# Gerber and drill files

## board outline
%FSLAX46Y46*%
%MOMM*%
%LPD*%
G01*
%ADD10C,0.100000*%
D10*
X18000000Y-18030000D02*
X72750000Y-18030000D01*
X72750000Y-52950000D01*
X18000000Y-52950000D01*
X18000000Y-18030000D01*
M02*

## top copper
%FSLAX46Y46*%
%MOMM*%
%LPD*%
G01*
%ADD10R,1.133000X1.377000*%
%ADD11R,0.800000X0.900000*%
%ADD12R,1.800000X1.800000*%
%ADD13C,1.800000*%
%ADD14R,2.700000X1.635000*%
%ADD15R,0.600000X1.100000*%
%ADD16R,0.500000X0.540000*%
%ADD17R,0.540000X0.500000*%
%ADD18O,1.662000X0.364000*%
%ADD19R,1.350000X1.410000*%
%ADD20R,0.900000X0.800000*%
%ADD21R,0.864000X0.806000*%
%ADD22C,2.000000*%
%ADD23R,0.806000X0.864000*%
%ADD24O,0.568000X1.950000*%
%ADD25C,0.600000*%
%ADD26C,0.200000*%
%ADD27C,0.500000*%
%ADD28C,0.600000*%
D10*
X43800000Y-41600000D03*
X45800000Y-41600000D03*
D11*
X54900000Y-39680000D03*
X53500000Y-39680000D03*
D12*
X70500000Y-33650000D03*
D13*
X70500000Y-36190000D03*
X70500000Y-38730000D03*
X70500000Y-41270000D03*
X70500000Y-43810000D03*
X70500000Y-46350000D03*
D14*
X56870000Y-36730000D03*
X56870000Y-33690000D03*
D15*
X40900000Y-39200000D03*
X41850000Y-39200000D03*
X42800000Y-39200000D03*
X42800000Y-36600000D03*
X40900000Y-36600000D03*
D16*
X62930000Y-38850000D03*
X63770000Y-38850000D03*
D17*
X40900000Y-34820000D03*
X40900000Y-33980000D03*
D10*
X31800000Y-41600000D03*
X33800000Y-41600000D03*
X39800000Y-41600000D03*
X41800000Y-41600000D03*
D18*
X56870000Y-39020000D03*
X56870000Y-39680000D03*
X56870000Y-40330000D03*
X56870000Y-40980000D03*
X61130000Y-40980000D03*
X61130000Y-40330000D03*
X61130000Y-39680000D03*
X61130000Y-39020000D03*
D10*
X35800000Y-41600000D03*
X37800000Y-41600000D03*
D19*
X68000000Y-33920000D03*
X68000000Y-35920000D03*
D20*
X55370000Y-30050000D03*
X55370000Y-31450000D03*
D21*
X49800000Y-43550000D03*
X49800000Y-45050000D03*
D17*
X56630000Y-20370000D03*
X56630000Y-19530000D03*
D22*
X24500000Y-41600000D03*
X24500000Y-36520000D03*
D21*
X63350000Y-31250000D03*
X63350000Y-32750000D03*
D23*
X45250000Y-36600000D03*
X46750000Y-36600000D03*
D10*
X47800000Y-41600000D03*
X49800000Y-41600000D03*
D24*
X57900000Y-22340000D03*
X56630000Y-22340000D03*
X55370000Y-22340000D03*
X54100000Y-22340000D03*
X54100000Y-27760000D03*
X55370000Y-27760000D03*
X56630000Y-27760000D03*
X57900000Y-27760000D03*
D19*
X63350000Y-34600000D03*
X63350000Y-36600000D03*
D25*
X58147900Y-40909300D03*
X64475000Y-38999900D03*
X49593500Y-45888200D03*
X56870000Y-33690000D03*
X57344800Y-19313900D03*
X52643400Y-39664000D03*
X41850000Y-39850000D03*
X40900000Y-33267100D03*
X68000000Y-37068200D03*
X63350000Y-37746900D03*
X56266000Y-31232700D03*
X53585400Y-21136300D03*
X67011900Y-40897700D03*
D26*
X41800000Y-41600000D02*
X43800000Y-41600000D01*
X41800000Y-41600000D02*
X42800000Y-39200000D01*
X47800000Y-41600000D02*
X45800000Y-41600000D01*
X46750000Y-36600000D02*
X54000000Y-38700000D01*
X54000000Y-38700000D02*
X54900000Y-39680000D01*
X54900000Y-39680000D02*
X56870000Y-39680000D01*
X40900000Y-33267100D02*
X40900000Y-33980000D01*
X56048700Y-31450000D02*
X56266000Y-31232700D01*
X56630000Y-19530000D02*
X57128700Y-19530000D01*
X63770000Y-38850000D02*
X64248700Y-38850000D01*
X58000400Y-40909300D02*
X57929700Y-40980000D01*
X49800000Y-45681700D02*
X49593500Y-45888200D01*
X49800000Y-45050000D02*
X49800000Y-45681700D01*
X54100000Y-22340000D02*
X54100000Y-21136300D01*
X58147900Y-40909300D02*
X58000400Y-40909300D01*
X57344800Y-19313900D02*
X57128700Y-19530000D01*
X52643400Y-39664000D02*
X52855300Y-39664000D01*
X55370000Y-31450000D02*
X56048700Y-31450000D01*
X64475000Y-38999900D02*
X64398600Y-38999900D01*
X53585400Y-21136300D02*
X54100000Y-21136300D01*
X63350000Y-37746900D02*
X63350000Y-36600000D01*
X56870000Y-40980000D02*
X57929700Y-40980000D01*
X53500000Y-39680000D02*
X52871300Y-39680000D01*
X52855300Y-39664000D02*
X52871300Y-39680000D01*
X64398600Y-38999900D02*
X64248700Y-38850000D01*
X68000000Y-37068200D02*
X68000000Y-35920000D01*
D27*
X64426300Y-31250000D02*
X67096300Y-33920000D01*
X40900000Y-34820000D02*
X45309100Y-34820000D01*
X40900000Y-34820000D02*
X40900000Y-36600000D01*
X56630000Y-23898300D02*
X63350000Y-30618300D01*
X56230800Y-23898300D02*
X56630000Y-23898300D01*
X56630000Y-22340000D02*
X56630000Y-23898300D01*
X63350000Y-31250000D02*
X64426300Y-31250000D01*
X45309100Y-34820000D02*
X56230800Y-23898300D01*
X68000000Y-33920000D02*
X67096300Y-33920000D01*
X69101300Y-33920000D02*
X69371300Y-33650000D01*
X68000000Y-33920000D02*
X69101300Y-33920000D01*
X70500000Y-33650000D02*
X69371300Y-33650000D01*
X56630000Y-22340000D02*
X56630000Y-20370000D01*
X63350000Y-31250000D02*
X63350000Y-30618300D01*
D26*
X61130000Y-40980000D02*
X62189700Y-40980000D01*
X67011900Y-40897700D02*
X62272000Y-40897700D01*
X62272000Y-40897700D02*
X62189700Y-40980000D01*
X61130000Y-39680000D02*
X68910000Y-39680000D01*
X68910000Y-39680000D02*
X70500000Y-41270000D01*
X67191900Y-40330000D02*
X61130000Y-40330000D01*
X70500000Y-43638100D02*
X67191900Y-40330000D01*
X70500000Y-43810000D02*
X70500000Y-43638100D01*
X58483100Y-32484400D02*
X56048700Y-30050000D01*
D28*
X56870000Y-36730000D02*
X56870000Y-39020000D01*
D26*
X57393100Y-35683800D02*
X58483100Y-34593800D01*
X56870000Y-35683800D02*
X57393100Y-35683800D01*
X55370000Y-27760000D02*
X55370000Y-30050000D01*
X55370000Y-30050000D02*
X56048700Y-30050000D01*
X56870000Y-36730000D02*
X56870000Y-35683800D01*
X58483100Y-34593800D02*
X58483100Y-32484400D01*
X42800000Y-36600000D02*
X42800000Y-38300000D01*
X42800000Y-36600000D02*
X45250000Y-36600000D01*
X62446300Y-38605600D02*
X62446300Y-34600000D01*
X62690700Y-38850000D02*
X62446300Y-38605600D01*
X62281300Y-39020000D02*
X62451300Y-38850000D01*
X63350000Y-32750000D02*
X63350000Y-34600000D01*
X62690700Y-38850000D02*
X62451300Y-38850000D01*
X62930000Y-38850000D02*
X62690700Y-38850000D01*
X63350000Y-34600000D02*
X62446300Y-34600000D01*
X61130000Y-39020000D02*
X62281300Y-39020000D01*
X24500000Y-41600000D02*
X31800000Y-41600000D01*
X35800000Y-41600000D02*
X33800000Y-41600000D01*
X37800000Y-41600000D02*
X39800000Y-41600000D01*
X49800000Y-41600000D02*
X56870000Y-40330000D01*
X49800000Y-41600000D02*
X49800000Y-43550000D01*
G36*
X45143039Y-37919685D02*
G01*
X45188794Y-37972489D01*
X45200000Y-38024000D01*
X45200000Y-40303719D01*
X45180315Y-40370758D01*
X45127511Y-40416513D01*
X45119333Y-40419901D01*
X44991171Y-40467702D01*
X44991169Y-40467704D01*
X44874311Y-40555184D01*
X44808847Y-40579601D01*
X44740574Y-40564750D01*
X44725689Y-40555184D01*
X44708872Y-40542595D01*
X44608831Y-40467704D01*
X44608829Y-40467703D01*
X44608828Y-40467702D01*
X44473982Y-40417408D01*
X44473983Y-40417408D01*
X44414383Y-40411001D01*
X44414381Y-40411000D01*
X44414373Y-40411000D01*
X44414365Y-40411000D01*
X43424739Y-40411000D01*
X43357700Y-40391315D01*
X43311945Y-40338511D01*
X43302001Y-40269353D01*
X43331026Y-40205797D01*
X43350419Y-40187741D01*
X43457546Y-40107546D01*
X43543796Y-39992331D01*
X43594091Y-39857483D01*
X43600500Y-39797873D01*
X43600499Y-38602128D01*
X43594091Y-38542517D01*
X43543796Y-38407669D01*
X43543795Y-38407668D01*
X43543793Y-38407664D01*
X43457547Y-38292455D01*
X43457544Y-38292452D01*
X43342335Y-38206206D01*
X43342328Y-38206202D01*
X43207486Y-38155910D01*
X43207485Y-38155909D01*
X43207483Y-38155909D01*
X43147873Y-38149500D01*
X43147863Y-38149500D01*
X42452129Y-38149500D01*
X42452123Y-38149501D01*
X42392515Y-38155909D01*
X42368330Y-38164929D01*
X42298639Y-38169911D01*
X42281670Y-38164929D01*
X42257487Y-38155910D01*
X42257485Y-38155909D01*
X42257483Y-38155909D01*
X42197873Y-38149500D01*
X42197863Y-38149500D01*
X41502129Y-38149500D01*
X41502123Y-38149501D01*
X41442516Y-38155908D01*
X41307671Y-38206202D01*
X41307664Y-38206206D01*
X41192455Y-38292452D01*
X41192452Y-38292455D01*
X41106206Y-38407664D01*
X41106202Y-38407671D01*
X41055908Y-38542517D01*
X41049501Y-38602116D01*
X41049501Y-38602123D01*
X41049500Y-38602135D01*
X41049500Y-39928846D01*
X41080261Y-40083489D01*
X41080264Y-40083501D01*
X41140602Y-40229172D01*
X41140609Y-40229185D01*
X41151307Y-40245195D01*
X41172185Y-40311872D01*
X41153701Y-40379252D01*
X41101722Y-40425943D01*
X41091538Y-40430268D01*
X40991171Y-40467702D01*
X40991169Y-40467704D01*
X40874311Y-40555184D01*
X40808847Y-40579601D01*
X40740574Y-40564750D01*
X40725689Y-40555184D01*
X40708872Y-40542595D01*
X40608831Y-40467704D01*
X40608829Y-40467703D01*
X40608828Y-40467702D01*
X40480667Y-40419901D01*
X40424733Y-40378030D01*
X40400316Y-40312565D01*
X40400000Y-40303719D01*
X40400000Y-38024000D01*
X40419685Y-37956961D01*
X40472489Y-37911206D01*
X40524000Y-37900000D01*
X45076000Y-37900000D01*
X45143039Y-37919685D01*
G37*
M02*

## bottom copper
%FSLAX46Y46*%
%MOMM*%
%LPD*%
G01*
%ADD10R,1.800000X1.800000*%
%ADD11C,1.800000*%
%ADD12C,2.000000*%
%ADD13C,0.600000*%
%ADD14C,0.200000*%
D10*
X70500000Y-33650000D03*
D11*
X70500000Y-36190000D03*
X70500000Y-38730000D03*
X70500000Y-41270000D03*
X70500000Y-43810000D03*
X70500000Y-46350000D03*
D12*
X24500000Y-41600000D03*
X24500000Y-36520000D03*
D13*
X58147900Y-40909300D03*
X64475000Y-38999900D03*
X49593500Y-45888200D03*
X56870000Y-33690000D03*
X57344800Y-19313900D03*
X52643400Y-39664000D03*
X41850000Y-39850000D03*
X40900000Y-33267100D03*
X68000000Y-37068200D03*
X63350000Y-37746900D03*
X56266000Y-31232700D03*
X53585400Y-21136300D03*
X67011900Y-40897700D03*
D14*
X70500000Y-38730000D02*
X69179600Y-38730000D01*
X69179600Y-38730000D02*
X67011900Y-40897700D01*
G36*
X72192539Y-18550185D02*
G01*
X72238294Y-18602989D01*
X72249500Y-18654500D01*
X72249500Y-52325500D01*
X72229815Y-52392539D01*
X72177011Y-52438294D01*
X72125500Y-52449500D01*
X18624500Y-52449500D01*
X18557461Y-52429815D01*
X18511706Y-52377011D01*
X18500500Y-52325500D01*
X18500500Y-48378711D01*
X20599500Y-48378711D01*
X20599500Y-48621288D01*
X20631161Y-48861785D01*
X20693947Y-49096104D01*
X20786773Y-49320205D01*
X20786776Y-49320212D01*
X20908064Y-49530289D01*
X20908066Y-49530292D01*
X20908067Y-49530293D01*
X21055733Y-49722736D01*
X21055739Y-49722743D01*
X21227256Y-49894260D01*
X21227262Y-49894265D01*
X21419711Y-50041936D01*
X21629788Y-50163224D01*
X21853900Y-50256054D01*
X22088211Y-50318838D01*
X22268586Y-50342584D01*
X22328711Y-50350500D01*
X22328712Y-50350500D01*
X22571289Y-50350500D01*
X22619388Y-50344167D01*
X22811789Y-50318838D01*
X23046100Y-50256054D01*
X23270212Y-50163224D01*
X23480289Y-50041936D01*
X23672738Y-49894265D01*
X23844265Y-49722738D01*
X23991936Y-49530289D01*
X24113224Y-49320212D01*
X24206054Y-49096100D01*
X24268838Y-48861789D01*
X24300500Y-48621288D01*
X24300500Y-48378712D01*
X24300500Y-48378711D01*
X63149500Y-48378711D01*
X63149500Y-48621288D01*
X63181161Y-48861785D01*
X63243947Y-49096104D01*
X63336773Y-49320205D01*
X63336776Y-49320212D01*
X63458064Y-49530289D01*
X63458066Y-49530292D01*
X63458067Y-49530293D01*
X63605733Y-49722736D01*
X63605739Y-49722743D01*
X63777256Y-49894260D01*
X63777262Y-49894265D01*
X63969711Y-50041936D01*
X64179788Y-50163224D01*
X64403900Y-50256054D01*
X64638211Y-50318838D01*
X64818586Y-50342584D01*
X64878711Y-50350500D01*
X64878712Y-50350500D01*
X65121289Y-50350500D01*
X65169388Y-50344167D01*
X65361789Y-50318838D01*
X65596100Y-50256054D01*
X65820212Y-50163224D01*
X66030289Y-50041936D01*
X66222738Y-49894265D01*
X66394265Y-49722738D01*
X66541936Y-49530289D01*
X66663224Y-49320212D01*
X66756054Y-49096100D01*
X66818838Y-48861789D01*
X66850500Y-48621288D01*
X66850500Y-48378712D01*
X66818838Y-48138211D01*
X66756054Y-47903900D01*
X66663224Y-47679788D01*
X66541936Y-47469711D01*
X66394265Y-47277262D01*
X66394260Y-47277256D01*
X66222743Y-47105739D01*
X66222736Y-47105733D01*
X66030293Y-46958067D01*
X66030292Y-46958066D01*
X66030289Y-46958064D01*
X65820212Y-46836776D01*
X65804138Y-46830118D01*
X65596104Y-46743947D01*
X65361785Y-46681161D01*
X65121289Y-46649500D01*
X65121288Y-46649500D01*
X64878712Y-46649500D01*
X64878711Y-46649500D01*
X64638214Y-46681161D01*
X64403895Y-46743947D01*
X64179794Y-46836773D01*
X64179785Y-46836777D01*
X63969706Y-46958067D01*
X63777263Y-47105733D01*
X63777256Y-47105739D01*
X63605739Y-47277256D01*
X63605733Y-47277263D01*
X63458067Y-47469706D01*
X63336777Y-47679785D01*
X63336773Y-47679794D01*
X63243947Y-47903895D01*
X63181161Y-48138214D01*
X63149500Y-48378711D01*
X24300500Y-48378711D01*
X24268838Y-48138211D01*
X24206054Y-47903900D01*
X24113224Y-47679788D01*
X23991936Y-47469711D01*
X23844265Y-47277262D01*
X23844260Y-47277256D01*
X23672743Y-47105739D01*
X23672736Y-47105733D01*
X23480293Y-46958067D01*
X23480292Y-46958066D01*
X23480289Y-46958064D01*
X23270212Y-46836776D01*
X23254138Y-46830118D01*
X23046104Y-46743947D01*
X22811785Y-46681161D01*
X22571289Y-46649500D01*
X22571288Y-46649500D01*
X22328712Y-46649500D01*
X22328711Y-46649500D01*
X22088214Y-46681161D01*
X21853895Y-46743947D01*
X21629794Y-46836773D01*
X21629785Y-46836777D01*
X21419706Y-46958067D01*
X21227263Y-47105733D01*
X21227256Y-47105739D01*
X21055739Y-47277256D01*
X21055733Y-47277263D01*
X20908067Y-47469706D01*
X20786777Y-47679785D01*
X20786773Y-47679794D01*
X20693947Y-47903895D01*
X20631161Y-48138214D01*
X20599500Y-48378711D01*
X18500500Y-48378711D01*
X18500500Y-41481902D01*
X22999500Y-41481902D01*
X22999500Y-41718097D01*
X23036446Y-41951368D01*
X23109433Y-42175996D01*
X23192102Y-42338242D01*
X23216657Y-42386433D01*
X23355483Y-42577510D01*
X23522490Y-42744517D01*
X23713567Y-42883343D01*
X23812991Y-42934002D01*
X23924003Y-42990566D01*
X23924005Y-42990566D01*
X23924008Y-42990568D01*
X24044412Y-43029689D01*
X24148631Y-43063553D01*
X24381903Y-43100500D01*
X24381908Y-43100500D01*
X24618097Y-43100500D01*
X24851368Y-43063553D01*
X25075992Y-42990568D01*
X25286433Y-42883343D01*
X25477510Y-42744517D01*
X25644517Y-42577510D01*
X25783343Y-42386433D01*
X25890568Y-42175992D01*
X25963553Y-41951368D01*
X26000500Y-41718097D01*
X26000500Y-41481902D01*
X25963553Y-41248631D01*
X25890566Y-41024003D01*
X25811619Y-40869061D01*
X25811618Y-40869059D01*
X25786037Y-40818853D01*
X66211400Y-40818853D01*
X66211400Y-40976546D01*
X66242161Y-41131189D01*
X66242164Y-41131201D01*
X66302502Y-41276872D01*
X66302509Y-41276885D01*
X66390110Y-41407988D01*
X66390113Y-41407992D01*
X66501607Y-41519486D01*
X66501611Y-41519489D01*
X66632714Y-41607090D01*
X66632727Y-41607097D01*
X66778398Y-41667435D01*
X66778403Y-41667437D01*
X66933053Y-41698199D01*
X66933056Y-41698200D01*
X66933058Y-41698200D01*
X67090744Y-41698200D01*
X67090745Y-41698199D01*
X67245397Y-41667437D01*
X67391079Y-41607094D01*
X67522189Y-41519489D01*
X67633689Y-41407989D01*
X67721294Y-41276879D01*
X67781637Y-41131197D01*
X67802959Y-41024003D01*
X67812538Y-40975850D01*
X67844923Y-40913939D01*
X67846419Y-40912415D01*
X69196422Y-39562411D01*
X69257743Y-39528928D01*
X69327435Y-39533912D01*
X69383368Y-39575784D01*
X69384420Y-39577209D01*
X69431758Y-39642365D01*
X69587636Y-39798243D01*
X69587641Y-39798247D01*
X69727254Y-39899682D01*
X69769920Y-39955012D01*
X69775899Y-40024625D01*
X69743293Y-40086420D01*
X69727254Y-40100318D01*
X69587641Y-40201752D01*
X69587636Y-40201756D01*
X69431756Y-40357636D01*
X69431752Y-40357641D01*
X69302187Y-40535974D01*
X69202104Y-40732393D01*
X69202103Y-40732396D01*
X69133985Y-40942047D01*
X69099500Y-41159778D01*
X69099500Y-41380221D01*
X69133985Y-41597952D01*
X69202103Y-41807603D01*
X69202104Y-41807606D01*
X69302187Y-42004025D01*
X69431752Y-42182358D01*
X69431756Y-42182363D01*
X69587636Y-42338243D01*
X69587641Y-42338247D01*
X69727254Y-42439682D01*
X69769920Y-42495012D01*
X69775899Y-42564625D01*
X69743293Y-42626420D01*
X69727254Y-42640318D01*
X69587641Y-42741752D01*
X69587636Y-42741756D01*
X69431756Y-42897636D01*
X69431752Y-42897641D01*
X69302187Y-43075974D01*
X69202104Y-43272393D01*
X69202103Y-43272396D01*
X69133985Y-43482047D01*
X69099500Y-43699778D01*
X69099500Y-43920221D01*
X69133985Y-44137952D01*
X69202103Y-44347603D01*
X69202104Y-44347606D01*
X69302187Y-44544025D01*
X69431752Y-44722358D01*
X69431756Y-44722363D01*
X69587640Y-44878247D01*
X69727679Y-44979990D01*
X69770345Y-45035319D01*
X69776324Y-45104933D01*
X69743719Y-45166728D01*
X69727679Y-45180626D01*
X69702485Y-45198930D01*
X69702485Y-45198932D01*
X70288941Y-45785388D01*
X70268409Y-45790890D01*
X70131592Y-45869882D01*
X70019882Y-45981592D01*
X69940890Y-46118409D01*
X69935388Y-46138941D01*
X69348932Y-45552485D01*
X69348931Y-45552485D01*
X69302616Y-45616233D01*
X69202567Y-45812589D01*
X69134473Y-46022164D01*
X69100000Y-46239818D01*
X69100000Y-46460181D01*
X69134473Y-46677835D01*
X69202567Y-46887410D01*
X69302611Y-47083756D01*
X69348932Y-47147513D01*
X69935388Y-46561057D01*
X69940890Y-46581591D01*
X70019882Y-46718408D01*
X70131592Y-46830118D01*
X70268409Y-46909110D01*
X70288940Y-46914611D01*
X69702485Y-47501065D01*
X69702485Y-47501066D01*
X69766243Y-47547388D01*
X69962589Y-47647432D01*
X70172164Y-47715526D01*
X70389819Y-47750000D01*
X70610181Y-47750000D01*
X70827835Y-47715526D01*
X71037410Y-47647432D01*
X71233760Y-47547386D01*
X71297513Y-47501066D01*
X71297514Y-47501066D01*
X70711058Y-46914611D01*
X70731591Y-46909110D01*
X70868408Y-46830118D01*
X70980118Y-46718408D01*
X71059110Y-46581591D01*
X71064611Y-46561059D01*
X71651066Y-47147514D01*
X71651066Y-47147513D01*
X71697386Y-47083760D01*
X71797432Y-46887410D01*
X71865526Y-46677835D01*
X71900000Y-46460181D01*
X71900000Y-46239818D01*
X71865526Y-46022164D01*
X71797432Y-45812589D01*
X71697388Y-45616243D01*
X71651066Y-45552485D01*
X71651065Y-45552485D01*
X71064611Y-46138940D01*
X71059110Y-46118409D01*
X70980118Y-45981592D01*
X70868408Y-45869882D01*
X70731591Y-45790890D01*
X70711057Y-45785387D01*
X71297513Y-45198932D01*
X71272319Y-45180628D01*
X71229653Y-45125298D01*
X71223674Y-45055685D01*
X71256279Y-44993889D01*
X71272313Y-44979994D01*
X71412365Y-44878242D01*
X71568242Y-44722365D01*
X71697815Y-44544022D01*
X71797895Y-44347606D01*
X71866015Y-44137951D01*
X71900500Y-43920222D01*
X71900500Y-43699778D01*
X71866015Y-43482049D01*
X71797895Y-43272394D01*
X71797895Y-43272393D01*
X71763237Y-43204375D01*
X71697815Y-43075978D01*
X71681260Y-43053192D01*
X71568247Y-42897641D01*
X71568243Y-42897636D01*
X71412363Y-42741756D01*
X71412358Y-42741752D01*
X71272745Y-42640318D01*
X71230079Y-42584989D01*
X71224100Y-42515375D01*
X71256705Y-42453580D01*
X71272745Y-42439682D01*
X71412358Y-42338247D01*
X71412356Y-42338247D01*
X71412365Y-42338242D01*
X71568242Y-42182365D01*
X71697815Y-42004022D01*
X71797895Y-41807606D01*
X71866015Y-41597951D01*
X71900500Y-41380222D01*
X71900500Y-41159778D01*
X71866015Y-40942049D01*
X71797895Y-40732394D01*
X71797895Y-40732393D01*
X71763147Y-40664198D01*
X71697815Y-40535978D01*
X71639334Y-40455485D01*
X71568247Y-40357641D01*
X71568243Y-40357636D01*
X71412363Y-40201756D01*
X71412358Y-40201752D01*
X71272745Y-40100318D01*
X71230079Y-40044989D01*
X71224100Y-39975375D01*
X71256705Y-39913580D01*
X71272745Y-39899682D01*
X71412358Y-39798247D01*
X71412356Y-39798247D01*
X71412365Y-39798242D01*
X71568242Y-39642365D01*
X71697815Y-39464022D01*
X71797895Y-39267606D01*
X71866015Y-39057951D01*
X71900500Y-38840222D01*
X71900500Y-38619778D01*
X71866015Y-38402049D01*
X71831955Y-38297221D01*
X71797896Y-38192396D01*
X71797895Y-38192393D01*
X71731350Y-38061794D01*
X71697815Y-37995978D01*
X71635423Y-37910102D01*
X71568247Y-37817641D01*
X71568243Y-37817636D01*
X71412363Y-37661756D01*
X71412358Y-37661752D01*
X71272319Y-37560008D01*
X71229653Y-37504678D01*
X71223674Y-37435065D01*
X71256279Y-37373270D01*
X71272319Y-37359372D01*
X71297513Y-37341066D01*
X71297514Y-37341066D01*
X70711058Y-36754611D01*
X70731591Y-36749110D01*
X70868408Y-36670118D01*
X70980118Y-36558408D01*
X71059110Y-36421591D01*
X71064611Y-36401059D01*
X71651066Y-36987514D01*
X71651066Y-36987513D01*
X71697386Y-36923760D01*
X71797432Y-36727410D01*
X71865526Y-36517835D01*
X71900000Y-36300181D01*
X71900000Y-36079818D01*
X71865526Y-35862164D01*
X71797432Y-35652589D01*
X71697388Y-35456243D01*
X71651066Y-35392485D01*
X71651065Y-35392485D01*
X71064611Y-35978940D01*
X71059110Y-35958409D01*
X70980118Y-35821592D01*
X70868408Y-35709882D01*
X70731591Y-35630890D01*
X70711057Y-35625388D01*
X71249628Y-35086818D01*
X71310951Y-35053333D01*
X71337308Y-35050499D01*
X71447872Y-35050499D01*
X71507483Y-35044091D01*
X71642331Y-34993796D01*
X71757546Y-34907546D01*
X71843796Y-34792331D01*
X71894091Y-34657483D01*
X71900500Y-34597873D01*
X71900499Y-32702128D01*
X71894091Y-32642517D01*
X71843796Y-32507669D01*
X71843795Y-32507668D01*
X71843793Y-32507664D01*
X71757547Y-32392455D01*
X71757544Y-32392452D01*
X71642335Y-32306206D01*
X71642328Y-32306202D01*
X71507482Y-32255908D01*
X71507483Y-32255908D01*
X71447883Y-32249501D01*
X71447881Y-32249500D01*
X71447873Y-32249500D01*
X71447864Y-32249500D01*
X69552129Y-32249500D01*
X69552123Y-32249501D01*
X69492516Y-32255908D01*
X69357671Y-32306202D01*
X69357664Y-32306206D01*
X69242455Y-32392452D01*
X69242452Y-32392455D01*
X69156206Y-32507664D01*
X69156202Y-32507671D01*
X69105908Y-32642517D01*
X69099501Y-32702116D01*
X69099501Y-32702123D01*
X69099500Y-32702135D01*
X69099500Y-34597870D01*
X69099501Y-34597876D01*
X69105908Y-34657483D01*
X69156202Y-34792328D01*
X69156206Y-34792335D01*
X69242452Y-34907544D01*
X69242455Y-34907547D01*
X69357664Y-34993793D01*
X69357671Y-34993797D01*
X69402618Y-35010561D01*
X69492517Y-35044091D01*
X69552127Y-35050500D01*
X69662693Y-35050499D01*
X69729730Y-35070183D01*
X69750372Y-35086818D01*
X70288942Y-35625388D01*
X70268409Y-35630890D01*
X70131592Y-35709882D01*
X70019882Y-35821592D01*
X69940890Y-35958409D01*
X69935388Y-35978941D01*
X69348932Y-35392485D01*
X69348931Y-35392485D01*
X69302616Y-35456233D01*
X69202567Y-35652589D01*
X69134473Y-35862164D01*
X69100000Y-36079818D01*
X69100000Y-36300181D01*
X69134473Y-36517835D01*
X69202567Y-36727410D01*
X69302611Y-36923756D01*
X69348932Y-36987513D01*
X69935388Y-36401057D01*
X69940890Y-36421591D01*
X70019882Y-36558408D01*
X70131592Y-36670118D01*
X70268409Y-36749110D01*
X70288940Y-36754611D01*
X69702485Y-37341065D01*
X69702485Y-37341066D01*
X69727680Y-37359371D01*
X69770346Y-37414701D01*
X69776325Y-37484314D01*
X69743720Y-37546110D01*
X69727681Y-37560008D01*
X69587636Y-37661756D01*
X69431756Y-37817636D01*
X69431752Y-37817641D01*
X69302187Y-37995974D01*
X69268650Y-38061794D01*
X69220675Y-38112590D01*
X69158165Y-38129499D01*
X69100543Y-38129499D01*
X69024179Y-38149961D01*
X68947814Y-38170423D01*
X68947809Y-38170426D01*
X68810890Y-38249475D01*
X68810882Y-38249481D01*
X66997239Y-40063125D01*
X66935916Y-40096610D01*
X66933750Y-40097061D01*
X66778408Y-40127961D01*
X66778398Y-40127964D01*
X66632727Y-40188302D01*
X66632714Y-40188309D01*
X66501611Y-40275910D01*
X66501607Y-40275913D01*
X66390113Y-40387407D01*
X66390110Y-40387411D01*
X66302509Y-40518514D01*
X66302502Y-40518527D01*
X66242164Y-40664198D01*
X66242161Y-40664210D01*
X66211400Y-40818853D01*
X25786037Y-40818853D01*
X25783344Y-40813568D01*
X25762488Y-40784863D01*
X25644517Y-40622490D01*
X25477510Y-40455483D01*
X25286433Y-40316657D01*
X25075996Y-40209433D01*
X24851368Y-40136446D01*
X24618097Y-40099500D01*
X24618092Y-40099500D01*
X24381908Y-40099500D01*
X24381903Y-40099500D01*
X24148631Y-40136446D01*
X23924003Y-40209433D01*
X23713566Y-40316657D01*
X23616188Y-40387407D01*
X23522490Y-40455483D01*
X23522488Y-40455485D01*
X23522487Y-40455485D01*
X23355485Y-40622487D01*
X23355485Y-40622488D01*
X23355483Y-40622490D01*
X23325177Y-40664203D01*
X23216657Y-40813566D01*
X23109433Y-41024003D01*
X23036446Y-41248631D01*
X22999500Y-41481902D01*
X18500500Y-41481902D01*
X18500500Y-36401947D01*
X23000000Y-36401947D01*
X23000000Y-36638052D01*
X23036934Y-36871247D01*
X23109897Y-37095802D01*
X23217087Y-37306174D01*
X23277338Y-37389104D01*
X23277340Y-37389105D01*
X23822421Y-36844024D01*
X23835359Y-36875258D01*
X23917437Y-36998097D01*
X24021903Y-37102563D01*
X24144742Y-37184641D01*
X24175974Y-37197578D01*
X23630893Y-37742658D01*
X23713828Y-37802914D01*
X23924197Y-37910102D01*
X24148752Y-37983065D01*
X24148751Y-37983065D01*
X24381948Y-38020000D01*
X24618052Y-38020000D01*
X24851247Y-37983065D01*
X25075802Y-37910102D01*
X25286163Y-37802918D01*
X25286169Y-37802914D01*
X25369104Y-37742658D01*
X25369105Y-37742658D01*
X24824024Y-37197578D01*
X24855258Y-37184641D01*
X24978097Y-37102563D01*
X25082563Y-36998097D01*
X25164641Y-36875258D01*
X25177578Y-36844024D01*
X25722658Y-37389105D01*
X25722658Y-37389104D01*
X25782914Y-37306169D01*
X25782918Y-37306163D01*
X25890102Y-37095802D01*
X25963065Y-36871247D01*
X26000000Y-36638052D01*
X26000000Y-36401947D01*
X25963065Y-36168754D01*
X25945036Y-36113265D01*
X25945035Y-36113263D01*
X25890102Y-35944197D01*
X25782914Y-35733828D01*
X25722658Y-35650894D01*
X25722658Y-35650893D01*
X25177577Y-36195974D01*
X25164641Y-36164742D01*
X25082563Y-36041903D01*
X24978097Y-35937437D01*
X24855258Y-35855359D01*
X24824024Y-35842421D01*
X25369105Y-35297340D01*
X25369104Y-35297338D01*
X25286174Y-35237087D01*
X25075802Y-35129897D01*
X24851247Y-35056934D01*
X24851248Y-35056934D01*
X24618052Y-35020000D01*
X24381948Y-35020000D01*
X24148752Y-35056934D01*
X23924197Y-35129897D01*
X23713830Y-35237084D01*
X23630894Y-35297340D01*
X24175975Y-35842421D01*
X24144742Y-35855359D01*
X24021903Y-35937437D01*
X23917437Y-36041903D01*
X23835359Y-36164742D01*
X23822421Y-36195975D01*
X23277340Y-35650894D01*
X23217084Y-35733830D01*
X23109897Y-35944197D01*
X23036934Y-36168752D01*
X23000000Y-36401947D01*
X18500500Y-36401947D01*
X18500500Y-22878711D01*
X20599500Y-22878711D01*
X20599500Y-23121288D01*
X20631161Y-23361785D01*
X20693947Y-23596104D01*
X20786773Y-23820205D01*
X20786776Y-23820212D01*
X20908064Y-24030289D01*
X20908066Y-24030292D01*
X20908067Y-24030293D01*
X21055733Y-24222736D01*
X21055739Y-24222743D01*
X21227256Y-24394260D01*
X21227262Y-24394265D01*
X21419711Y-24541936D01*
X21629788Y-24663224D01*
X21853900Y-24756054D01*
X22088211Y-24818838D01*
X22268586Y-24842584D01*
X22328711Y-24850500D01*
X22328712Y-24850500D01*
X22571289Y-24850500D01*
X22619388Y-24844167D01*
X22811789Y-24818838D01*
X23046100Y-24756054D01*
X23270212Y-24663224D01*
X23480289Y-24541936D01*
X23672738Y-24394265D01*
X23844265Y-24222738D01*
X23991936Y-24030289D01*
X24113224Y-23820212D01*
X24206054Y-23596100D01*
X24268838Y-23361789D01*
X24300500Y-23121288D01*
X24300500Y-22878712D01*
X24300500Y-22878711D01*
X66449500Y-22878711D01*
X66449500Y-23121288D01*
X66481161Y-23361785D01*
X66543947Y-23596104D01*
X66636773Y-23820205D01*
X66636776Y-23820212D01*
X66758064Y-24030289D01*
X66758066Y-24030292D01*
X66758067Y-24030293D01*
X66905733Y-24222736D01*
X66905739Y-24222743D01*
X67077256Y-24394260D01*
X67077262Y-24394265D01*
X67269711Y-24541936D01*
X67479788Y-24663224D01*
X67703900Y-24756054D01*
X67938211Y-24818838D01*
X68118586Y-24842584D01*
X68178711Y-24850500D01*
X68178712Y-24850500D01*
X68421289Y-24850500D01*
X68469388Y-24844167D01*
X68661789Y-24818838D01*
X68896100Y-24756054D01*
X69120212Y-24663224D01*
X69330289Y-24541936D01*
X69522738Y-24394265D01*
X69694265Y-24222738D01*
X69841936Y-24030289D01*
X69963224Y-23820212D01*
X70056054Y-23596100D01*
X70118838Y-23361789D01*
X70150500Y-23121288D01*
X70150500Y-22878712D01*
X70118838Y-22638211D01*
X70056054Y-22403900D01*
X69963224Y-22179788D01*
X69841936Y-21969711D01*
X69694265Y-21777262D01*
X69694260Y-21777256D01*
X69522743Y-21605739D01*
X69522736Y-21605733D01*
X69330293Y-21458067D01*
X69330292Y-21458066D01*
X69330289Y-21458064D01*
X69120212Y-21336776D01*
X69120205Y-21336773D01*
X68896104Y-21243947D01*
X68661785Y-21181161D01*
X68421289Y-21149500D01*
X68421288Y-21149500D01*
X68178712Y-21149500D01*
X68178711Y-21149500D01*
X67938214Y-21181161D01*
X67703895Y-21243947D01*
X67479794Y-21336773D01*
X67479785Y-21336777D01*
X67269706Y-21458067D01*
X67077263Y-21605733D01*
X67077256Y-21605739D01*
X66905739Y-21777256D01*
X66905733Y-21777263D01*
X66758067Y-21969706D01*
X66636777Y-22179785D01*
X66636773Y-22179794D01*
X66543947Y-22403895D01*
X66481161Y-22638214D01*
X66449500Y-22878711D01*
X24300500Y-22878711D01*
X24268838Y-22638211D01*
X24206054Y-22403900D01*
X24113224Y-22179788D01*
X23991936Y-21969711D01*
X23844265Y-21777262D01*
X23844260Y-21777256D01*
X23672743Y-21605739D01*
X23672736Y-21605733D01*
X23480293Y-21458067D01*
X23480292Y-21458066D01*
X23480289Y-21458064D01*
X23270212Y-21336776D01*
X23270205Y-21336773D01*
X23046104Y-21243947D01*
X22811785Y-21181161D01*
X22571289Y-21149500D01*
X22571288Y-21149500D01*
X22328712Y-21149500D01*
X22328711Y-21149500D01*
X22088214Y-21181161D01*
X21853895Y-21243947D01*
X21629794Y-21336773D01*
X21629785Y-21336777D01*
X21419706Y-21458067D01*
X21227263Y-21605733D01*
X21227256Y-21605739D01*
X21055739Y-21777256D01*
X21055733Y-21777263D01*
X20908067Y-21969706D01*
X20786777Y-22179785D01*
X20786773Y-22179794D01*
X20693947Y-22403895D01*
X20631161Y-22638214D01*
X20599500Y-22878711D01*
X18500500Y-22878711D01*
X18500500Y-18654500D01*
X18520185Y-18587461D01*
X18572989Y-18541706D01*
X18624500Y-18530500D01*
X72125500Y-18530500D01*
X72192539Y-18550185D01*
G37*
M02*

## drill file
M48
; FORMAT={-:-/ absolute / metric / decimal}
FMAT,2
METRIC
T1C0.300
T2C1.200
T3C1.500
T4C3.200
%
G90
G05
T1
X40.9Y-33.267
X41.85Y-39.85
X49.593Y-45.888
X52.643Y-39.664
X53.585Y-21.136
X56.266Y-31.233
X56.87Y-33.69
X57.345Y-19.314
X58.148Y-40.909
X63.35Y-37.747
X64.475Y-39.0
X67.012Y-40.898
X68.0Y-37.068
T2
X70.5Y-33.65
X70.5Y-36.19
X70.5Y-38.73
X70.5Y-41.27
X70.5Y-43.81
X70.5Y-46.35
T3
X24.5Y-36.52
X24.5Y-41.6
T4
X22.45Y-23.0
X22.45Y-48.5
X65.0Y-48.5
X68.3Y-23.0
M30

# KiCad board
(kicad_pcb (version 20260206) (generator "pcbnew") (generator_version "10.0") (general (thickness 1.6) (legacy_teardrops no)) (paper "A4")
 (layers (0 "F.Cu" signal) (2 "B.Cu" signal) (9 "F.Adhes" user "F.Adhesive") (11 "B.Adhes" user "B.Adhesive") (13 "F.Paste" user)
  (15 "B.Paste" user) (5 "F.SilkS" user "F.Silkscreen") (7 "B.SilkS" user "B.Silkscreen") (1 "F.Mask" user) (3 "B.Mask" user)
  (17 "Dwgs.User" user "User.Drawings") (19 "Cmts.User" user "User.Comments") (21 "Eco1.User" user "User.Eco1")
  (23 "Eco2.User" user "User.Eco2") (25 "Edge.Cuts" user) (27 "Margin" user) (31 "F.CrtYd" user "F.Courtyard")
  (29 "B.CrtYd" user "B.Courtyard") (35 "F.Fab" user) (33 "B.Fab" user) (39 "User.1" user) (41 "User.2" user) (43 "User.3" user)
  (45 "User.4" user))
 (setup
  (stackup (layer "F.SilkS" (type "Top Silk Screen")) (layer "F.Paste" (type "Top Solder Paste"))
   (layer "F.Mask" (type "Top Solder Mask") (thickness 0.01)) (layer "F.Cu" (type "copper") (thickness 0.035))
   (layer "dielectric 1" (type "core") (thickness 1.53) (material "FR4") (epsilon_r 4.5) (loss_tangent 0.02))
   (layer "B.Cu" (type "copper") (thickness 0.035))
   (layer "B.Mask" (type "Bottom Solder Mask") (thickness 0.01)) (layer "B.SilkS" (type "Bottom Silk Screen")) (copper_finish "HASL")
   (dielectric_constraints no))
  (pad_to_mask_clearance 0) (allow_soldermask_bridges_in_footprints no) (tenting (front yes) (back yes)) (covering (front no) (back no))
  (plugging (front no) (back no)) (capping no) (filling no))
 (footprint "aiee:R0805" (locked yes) (layer "F.Cu") (at 44.8 41.6)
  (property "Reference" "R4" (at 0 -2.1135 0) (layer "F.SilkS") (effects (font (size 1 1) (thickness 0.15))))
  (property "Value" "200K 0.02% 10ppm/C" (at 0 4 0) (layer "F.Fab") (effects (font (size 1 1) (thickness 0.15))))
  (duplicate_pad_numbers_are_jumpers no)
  (pad "1" smd rect (at -1 0) (size 1.133 1.377) (layers "F.Cu" "F.Mask" "F.Paste") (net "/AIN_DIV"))
  (pad "2" smd rect (at 1 0) (size 1.133 1.377) (layers "F.Cu" "F.Mask" "F.Paste") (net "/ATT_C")))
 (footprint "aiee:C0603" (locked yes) (layer "F.Cu") (at 54.2 39.68 180)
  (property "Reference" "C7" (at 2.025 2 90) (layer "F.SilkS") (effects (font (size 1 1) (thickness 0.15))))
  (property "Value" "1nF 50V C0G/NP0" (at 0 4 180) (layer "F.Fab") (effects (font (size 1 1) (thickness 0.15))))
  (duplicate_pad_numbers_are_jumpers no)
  (pad "1" smd rect (at -0.7 0 180) (size 0.8 0.9) (layers "F.Cu" "F.Mask" "F.Paste") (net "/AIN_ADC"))
  (pad "2" smd rect (at 0.7 0 180) (size 0.8 0.9) (layers "F.Cu" "F.Mask" "F.Paste") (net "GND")))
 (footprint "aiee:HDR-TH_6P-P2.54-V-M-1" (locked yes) (layer "F.Cu") (at 70.5 40 -90)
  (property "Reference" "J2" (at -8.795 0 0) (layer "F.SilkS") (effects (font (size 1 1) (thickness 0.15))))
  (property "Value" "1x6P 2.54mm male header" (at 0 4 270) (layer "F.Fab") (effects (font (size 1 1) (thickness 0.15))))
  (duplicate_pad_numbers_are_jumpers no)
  (pad "1" thru_hole rect (at -6.35 0 270) (size 1.8 1.8) (drill 1.199998) (layers "*.Cu" "*.Mask") (remove_unused_layers no) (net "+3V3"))
  (pad "2" thru_hole circle (at -3.81 0 270) (size 1.8 1.8) (drill 1.199998) (layers "*.Cu" "*.Mask") (remove_unused_layers no) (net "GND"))
  (pad "3" thru_hole circle (at -1.27 0 270) (size 1.8 1.8) (drill 1.199998) (layers "*.Cu" "*.Mask") (remove_unused_layers no) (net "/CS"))
  (pad "4" thru_hole circle (at 1.27 0 270) (size 1.8 1.8) (drill 1.199998) (layers "*.Cu" "*.Mask") (remove_unused_layers no) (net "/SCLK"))
  (pad "5" thru_hole circle (at 3.81 0 270) (size 1.8 1.8) (drill 1.199998) (layers "*.Cu" "*.Mask") (remove_unused_layers no) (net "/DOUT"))
  (pad "6" thru_hole circle (at 6.35 0 270) (size 1.8 1.8) (drill 1.199998) (layers "*.Cu" "*.Mask") (remove_unused_layers no) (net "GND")))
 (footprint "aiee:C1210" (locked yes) (layer "F.Cu") (at 56.87 35.21 90)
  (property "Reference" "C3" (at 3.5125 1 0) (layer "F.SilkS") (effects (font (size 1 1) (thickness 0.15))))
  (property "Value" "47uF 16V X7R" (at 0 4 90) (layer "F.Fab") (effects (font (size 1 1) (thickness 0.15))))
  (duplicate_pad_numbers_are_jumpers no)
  (pad "1" smd rect (at -1.52 0 90) (size 1.635 2.7) (layers "F.Cu" "F.Mask" "F.Paste") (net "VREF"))
  (pad "2" smd rect (at 1.52 0 90) (size 1.635 2.7) (layers "F.Cu" "F.Mask" "F.Paste") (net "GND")))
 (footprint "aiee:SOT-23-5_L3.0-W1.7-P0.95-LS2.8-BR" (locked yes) (layer "F.Cu") (at 41.85 37.9 -90)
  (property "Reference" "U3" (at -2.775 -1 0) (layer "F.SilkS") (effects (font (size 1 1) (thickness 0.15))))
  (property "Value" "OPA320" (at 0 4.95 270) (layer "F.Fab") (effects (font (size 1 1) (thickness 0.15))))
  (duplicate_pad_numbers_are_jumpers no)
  (pad "1" smd rect (at 1.3 0.95 270) (size 1.1 0.6) (layers "F.Cu" "F.Mask" "F.Paste") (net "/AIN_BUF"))
  (pad "2" smd rect (at 1.3 0 270) (size 1.1 0.6) (layers "F.Cu" "F.Mask" "F.Paste") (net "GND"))
  (pad "3" smd rect (at 1.3 -0.95 270) (size 1.1 0.6) (layers "F.Cu" "F.Mask" "F.Paste") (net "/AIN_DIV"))
  (pad "4" smd rect (at -1.3 -0.95 270) (size 1.1 0.6) (layers "F.Cu" "F.Mask" "F.Paste") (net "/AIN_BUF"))
  (pad "5" smd rect (at -1.3 0.95 270) (size 1.1 0.6) (layers "F.Cu" "F.Mask" "F.Paste") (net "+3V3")))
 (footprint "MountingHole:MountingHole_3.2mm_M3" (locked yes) (layer "F.Cu") (at 68.3 23)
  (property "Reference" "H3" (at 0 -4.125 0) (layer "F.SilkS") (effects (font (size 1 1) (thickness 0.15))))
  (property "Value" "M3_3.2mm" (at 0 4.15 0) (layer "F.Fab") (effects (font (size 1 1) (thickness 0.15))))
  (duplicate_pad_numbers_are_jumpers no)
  (pad "" np_thru_hole circle (at 0 0) (size 3.2 3.2) (drill 3.2) (layers "*.Cu" "*.Mask")))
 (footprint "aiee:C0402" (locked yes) (layer "F.Cu") (at 63.35 38.85)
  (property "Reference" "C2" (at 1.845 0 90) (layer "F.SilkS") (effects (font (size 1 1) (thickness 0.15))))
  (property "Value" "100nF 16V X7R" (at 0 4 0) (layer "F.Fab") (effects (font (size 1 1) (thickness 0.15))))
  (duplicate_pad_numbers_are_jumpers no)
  (pad "1" smd rect (at -0.42 0) (size 0.5 0.54) (layers "F.Cu" "F.Mask" "F.Paste") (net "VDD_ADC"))
  (pad "2" smd rect (at 0.42 0) (size 0.5 0.54) (layers "F.Cu" "F.Mask" "F.Paste") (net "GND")))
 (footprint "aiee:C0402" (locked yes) (layer "F.Cu") (at 40.9 34.4 90)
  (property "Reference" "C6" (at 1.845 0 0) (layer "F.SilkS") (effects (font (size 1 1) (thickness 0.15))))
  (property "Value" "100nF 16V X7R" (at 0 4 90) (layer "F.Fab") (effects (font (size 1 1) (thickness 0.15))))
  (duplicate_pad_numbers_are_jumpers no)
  (pad "1" smd rect (at -0.42 0 90) (size 0.5 0.54) (layers "F.Cu" "F.Mask" "F.Paste") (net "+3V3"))
  (pad "2" smd rect (at 0.42 0 90) (size 0.5 0.54) (layers "F.Cu" "F.Mask" "F.Paste") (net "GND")))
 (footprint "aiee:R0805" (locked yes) (layer "F.Cu") (at 32.8 41.6)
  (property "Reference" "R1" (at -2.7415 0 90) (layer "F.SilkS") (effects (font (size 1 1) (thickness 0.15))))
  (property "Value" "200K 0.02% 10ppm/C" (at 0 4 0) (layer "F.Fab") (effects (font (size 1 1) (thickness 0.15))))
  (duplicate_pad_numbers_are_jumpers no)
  (pad "1" smd rect (at -1 0) (size 1.133 1.377) (layers "F.Cu" "F.Mask" "F.Paste") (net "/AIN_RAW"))
  (pad "2" smd rect (at 1 0) (size 1.133 1.377) (layers "F.Cu" "F.Mask" "F.Paste") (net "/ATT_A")))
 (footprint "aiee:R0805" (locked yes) (layer "F.Cu") (at 40.8 41.6)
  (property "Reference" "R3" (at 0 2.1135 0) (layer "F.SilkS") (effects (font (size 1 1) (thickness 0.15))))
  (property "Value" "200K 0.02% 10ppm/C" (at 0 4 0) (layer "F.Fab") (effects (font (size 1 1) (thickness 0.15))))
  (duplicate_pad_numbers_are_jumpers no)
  (pad "1" smd rect (at -1 0) (size 1.133 1.377) (layers "F.Cu" "F.Mask" "F.Paste") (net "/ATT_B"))
  (pad "2" smd rect (at 1 0) (size 1.133 1.377) (layers "F.Cu" "F.Mask" "F.Paste") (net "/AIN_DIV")))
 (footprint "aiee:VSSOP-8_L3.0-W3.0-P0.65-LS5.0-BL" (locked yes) (layer "F.Cu") (at 59 40 -90)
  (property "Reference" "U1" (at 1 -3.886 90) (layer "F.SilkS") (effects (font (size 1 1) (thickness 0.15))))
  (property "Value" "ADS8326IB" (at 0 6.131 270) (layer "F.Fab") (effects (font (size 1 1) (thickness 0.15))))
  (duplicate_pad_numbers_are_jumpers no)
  (pad "1" smd oval (at -0.98 2.13 270) (size 0.364 1.662) (layers "F.Cu" "F.Mask" "F.Paste") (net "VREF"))
  (pad "2" smd oval (at -0.32 2.13 270) (size 0.364 1.662) (layers "F.Cu" "F.Mask" "F.Paste") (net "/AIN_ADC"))
  (pad "3" smd oval (at 0.33 2.13 270) (size 0.364 1.662) (layers "F.Cu" "F.Mask" "F.Paste") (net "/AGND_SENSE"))
  (pad "4" smd oval (at 0.98 2.13 270) (size 0.364 1.662) (layers "F.Cu" "F.Mask" "F.Paste") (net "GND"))
  (pad "5" smd oval (at 0.98 -2.13 270) (size 0.364 1.662) (layers "F.Cu" "F.Mask" "F.Paste") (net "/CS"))
  (pad "6" smd oval (at 0.33 -2.13 270) (size 0.364 1.662) (layers "F.Cu" "F.Mask" "F.Paste") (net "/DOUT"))
  (pad "7" smd oval (at -0.32 -2.13 270) (size 0.364 1.662) (layers "F.Cu" "F.Mask" "F.Paste") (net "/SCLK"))
  (pad "8" smd oval (at -0.98 -2.13 270) (size 0.364 1.662) (layers "F.Cu" "F.Mask" "F.Paste") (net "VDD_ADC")))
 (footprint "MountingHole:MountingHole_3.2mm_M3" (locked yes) (layer "F.Cu") (at 22.45 23)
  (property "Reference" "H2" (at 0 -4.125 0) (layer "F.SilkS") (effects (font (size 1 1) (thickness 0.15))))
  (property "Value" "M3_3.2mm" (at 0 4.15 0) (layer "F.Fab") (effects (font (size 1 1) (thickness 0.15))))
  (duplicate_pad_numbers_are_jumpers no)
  (pad "" np_thru_hole circle (at 0 0) (size 3.2 3.2) (drill 3.2) (layers "*.Cu" "*.Mask")))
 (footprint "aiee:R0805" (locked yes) (layer "F.Cu") (at 36.8 41.6)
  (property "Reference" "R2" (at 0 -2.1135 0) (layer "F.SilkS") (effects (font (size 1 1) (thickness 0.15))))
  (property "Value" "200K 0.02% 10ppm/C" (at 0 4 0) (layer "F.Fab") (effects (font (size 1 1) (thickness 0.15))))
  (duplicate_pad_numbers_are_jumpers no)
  (pad "1" smd rect (at -1 0) (size 1.133 1.377) (layers "F.Cu" "F.Mask" "F.Paste") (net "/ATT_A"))
  (pad "2" smd rect (at 1 0) (size 1.133 1.377) (layers "F.Cu" "F.Mask" "F.Paste") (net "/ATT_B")))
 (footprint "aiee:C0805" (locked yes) (layer "F.Cu") (at 68 34.92 -90)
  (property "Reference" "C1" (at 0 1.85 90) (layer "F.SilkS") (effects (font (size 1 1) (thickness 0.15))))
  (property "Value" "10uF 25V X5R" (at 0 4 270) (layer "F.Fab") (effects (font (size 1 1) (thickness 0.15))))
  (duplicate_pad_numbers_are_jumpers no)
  (pad "1" smd rect (at -1 0 270) (size 1.41 1.35) (layers "F.Cu" "F.Mask" "F.Paste") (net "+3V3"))
  (pad "2" smd rect (at 1 0 270) (size 1.41 1.35) (layers "F.Cu" "F.Mask" "F.Paste") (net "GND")))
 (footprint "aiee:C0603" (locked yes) (layer "F.Cu") (at 55.37 30.75 -90)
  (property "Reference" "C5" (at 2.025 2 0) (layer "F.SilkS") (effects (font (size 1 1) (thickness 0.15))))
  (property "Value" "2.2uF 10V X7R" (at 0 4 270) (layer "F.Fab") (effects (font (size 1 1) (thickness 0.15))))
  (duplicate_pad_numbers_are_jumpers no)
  (pad "1" smd rect (at -0.7 0 270) (size 0.8 0.9) (layers "F.Cu" "F.Mask" "F.Paste") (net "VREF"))
  (pad "2" smd rect (at 0.7 0 270) (size 0.8 0.9) (layers "F.Cu" "F.Mask" "F.Paste") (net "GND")))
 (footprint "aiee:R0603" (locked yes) (layer "F.Cu") (at 49.8 44.3 -90)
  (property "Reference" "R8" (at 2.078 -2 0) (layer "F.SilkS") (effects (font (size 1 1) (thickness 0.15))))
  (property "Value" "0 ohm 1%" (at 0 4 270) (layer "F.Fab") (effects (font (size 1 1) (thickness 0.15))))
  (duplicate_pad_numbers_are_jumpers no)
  (pad "1" smd rect (at -0.75 0 270) (size 0.806 0.864) (layers "F.Cu" "F.Mask" "F.Paste") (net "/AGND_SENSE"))
  (pad "2" smd rect (at 0.75 0 270) (size 0.806 0.864) (layers "F.Cu" "F.Mask" "F.Paste") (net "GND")))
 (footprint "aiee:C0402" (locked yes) (layer "F.Cu") (at 56.63 19.95 90)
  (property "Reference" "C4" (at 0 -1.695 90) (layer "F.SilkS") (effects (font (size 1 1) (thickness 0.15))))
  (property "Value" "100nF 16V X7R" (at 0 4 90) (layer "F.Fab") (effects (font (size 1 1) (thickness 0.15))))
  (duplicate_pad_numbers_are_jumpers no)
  (pad "1" smd rect (at -0.42 0 90) (size 0.5 0.54) (layers "F.Cu" "F.Mask" "F.Paste") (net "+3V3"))
  (pad "2" smd rect (at 0.42 0 90) (size 0.5 0.54) (layers "F.Cu" "F.Mask" "F.Paste") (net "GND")))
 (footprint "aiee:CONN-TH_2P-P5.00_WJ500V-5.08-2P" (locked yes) (layer "F.Cu") (at 24.5 39.06 90)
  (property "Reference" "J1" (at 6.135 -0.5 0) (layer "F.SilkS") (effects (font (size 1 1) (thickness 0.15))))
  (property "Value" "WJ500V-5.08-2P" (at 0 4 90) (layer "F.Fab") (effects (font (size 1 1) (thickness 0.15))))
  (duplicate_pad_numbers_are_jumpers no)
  (pad "1" thru_hole circle (at -2.54 0 270) (size 2 2) (drill 1.5) (layers "*.Cu" "*.Mask") (remove_unused_layers no) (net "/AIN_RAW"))
  (pad "2" thru_hole circle (at 2.54 0 270) (size 2 2) (drill 1.5) (layers "*.Cu" "*.Mask") (remove_unused_layers no) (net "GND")))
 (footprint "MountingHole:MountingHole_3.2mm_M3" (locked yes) (layer "F.Cu") (at 22.45 48.5)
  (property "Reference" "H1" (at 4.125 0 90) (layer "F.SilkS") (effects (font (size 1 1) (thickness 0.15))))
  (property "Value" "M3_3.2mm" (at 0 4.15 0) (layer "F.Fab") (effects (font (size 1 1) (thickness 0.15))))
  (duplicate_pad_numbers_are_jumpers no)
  (pad "" np_thru_hole circle (at 0 0) (size 3.2 3.2) (drill 3.2) (layers "*.Cu" "*.Mask")))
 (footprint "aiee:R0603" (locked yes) (layer "F.Cu") (at 63.35 32 -90)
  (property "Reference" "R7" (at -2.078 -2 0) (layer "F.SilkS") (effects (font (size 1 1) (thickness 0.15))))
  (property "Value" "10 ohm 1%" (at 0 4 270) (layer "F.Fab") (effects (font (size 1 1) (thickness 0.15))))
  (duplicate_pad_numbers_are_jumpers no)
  (pad "1" smd rect (at -0.75 0 270) (size 0.806 0.864) (layers "F.Cu" "F.Mask" "F.Paste") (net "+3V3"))
  (pad "2" smd rect (at 0.75 0 270) (size 0.806 0.864) (layers "F.Cu" "F.Mask" "F.Paste") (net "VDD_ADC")))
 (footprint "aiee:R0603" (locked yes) (layer "F.Cu") (at 46 36.6)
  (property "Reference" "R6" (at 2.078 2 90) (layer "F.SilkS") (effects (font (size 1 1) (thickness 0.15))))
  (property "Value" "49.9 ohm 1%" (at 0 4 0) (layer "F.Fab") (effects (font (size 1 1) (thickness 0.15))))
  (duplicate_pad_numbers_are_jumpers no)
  (pad "1" smd rect (at -0.75 0) (size 0.806 0.864) (layers "F.Cu" "F.Mask" "F.Paste") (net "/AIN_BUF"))
  (pad "2" smd rect (at 0.75 0) (size 0.806 0.864) (layers "F.Cu" "F.Mask" "F.Paste") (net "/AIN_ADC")))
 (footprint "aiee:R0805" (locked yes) (layer "F.Cu") (at 48.8 41.6)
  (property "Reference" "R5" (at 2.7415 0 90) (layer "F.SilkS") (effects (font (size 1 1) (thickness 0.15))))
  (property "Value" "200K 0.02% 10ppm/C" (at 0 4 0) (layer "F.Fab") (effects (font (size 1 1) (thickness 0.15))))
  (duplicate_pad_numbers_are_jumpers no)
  (pad "1" smd rect (at -1 0) (size 1.133 1.377) (layers "F.Cu" "F.Mask" "F.Paste") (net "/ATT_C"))
  (pad "2" smd rect (at 1 0) (size 1.133 1.377) (layers "F.Cu" "F.Mask" "F.Paste") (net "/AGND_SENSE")))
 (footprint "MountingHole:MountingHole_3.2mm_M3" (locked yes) (layer "F.Cu") (at 65 48.5)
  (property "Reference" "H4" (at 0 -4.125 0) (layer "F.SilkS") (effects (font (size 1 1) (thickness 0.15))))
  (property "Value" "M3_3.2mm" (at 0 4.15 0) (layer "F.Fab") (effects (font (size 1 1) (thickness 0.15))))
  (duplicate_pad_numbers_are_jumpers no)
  (pad "" np_thru_hole circle (at 0 0) (size 3.2 3.2) (drill 3.2) (layers "*.Cu" "*.Mask")))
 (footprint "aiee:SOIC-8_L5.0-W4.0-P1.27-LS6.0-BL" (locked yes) (layer "F.Cu") (at 56 25.05 180)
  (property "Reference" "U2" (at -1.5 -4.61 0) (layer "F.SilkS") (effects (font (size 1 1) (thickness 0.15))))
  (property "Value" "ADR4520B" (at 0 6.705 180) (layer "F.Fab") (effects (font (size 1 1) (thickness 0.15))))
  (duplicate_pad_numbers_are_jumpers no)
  (pad "1" smd oval (at -1.9 2.71 180) (size 0.568 1.95) (layers "F.Cu" "F.Mask" "F.Paste") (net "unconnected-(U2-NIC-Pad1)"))
  (pad "2" smd oval (at -0.63 2.71 180) (size 0.568 1.95) (layers "F.Cu" "F.Mask" "F.Paste") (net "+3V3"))
  (pad "3" smd oval (at 0.63 2.71 180) (size 0.568 1.95) (layers "F.Cu" "F.Mask" "F.Paste") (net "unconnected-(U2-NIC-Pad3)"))
  (pad "4" smd oval (at 1.9 2.71 180) (size 0.568 1.95) (layers "F.Cu" "F.Mask" "F.Paste") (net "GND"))
  (pad "5" smd oval (at 1.9 -2.71 180) (size 0.568 1.95) (layers "F.Cu" "F.Mask" "F.Paste") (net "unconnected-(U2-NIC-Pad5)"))
  (pad "6" smd oval (at 0.63 -2.71 180) (size 0.568 1.95) (layers "F.Cu" "F.Mask" "F.Paste") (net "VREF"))
  (pad "7" smd oval (at -0.63 -2.71 180) (size 0.568 1.95) (layers "F.Cu" "F.Mask" "F.Paste") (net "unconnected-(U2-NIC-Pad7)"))
  (pad "8" smd oval (at -1.9 -2.71 180) (size 0.568 1.95) (layers "F.Cu" "F.Mask" "F.Paste") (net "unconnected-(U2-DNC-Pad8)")))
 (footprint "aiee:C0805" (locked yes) (layer "F.Cu") (at 63.35 35.6 -90)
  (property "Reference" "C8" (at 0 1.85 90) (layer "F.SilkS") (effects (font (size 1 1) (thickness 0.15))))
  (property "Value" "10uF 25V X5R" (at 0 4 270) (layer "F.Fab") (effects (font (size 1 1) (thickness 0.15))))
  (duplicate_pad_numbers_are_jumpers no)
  (pad "1" smd rect (at -1 0 270) (size 1.41 1.35) (layers "F.Cu" "F.Mask" "F.Paste") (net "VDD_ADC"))
  (pad "2" smd rect (at 1 0 270) (size 1.41 1.35) (layers "F.Cu" "F.Mask" "F.Paste") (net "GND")))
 (gr_rect (start 18 18.03) (end 72.75 52.95) (stroke (width 0.1) (type default)) (fill no) (layer "Edge.Cuts"))
 (segment (start 41.8 41.6) (end 43.8 41.6) (width 0.2) (layer "F.Cu") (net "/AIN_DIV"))
 (segment (start 41.8 41.6) (end 42.8 39.2) (width 0.2) (layer "F.Cu") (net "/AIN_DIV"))
 (segment (start 47.8 41.6) (end 45.8 41.6) (width 0.2) (layer "F.Cu") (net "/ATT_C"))
 (segment (start 46.75 36.6) (end 54 38.7) (width 0.2) (layer "F.Cu") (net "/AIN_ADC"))
 (segment (start 54 38.7) (end 54.9 39.68) (width 0.2) (layer "F.Cu") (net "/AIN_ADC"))
 (segment (start 54.9 39.68) (end 56.87 39.68) (width 0.2) (layer "F.Cu") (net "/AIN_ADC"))
 (segment (start 40.9 33.2671) (end 40.9 33.98) (width 0.2) (layer "F.Cu") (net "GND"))
 (segment (start 56.0487 31.45) (end 56.266 31.2327) (width 0.2) (layer "F.Cu") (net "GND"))
 (segment (start 56.63 19.53) (end 57.1287 19.53) (width 0.2) (layer "F.Cu") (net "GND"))
 (segment (start 63.77 38.85) (end 64.2487 38.85) (width 0.2) (layer "F.Cu") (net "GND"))
 (segment (start 58.0004 40.9093) (end 57.9297 40.98) (width 0.2) (layer "F.Cu") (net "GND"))
 (segment (start 49.8 45.6817) (end 49.5935 45.8882) (width 0.2) (layer "F.Cu") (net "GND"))
 (segment (start 49.8 45.05) (end 49.8 45.6817) (width 0.2) (layer "F.Cu") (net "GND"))
 (segment (start 54.1 22.34) (end 54.1 21.1363) (width 0.2) (layer "F.Cu") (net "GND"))
 (segment (start 58.1479 40.9093) (end 58.0004 40.9093) (width 0.2) (layer "F.Cu") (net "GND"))
 (segment (start 57.3448 19.3139) (end 57.1287 19.53) (width 0.2) (layer "F.Cu") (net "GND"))
 (segment (start 52.6434 39.664) (end 52.8553 39.664) (width 0.2) (layer "F.Cu") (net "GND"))
 (segment (start 55.37 31.45) (end 56.0487 31.45) (width 0.2) (layer "F.Cu") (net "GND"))
 (segment (start 64.475 38.9999) (end 64.3986 38.9999) (width 0.2) (layer "F.Cu") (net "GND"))
 (segment (start 53.5854 21.1363) (end 54.1 21.1363) (width 0.2) (layer "F.Cu") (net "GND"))
 (segment (start 63.35 37.7469) (end 63.35 36.6) (width 0.2) (layer "F.Cu") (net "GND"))
 (segment (start 56.87 40.98) (end 57.9297 40.98) (width 0.2) (layer "F.Cu") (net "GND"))
 (segment (start 53.5 39.68) (end 52.8713 39.68) (width 0.2) (layer "F.Cu") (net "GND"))
 (segment (start 52.8553 39.664) (end 52.8713 39.68) (width 0.2) (layer "F.Cu") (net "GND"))
 (segment (start 64.3986 38.9999) (end 64.2487 38.85) (width 0.2) (layer "F.Cu") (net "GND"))
 (segment (start 68 37.0682) (end 68 35.92) (width 0.2) (layer "F.Cu") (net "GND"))
 (via (at 58.1479 40.9093) (size 0.6) (drill 0.3) (layers "F.Cu" "B.Cu") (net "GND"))
 (via (at 64.475 38.9999) (size 0.6) (drill 0.3) (layers "F.Cu" "B.Cu") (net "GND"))
 (via (at 49.5935 45.8882) (size 0.6) (drill 0.3) (layers "F.Cu" "B.Cu") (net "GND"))
 (via (at 56.87 33.69) (size 0.6) (drill 0.3) (layers "F.Cu" "B.Cu") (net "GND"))
 (via (at 57.3448 19.3139) (size 0.6) (drill 0.3) (layers "F.Cu" "B.Cu") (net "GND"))
 (via (at 52.6434 39.664) (size 0.6) (drill 0.3) (layers "F.Cu" "B.Cu") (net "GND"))
 (via (at 41.85 39.85) (size 0.6) (drill 0.3) (layers "F.Cu" "B.Cu") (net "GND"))
 (via (at 40.9 33.2671) (size 0.6) (drill 0.3) (layers "F.Cu" "B.Cu") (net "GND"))
 (via (at 68 37.0682) (size 0.6) (drill 0.3) (layers "F.Cu" "B.Cu") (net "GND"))
 (via (at 63.35 37.7469) (size 0.6) (drill 0.3) (layers "F.Cu" "B.Cu") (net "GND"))
 (via (at 56.266 31.2327) (size 0.6) (drill 0.3) (layers "F.Cu" "B.Cu") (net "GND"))
 (via (at 53.5854 21.1363) (size 0.6) (drill 0.3) (layers "F.Cu" "B.Cu") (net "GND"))
 (segment (start 64.4263 31.25) (end 67.0963 33.92) (width 0.5) (layer "F.Cu") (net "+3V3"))
 (segment (start 40.9 34.82) (end 45.3091 34.82) (width 0.5) (layer "F.Cu") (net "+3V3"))
 (segment (start 40.9 34.82) (end 40.9 36.6) (width 0.5) (layer "F.Cu") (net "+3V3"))
 (segment (start 56.63 23.8983) (end 63.35 30.6183) (width 0.5) (layer "F.Cu") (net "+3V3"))
 (segment (start 56.2308 23.8983) (end 56.63 23.8983) (width 0.5) (layer "F.Cu") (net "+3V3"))
 (segment (start 56.63 22.34) (end 56.63 23.8983) (width 0.5) (layer "F.Cu") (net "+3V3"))
 (segment (start 63.35 31.25) (end 64.4263 31.25) (width 0.5) (layer "F.Cu") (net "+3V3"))
 (segment (start 45.3091 34.82) (end 56.2308 23.8983) (width 0.5) (layer "F.Cu") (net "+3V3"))
 (segment (start 68 33.92) (end 67.0963 33.92) (width 0.5) (layer "F.Cu") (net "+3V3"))
 (segment (start 69.1013 33.92) (end 69.3713 33.65) (width 0.5) (layer "F.Cu") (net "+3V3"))
 (segment (start 68 33.92) (end 69.1013 33.92) (width 0.5) (layer "F.Cu") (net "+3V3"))
 (segment (start 70.5 33.65) (end 69.3713 33.65) (width 0.5) (layer "F.Cu") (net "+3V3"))
 (segment (start 56.63 22.34) (end 56.63 20.37) (width 0.5) (layer "F.Cu") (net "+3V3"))
 (segment (start 63.35 31.25) (end 63.35 30.6183) (width 0.5) (layer "F.Cu") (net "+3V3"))
 (segment (start 61.13 40.98) (end 62.1897 40.98) (width 0.2) (layer "F.Cu") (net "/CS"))
 (segment (start 67.0119 40.8977) (end 62.272 40.8977) (width 0.2) (layer "F.Cu") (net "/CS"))
 (segment (start 62.272 40.8977) (end 62.1897 40.98) (width 0.2) (layer "F.Cu") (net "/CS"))
 (via (at 67.0119 40.8977) (size 0.6) (drill 0.3) (layers "F.Cu" "B.Cu") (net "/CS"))
 (segment (start 70.5 38.73) (end 69.1796 38.73) (width 0.2) (layer "B.Cu") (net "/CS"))
 (segment (start 69.1796 38.73) (end 67.0119 40.8977) (width 0.2) (layer "B.Cu") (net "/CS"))
 (segment (start 61.13 39.68) (end 68.91 39.68) (width 0.2) (layer "F.Cu") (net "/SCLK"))
 (segment (start 68.91 39.68) (end 70.5 41.27) (width 0.2) (layer "F.Cu") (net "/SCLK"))
 (segment (start 67.1919 40.33) (end 61.13 40.33) (width 0.2) (layer "F.Cu") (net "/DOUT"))
 (segment (start 70.5 43.6381) (end 67.1919 40.33) (width 0.2) (layer "F.Cu") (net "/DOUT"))
 (segment (start 70.5 43.81) (end 70.5 43.6381) (width 0.2) (layer "F.Cu") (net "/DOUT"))
 (segment (start 58.4831 32.4844) (end 56.0487 30.05) (width 0.2) (layer "F.Cu") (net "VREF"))
 (segment (start 56.87 36.73) (end 56.87 39.02) (width 0.6) (layer "F.Cu") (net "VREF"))
 (segment (start 57.3931 35.6838) (end 58.4831 34.5938) (width 0.2) (layer "F.Cu") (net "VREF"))
 (segment (start 56.87 35.6838) (end 57.3931 35.6838) (width 0.2) (layer "F.Cu") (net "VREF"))
 (segment (start 55.37 27.76) (end 55.37 30.05) (width 0.2) (layer "F.Cu") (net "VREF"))
 (segment (start 55.37 30.05) (end 56.0487 30.05) (width 0.2) (layer "F.Cu") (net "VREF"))
 (segment (start 56.87 36.73) (end 56.87 35.6838) (width 0.2) (layer "F.Cu") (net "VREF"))
 (segment (start 58.4831 34.5938) (end 58.4831 32.4844) (width 0.2) (layer "F.Cu") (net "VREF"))
 (segment (start 42.8 36.6) (end 42.8 38.3) (width 0.2) (layer "F.Cu") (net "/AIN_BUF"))
 (segment (start 42.8 36.6) (end 45.25 36.6) (width 0.2) (layer "F.Cu") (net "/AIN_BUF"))
 (segment (start 62.4463 38.6056) (end 62.4463 34.6) (width 0.2) (layer "F.Cu") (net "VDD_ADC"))
 (segment (start 62.6907 38.85) (end 62.4463 38.6056) (width 0.2) (layer "F.Cu") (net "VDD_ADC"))
 (segment (start 62.2813 39.02) (end 62.4513 38.85) (width 0.2) (layer "F.Cu") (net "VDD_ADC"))
 (segment (start 63.35 32.75) (end 63.35 34.6) (width 0.2) (layer "F.Cu") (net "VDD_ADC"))
 (segment (start 62.6907 38.85) (end 62.4513 38.85) (width 0.2) (layer "F.Cu") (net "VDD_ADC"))
 (segment (start 62.93 38.85) (end 62.6907 38.85) (width 0.2) (layer "F.Cu") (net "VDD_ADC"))
 (segment (start 63.35 34.6) (end 62.4463 34.6) (width 0.2) (layer "F.Cu") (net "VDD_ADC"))
 (segment (start 61.13 39.02) (end 62.2813 39.02) (width 0.2) (layer "F.Cu") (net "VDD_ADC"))
 (segment (start 24.5 41.6) (end 31.8 41.6) (width 0.2) (layer "F.Cu") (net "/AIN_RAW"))
 (segment (start 35.8 41.6) (end 33.8 41.6) (width 0.2) (layer "F.Cu") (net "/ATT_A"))
 (segment (start 37.8 41.6) (end 39.8 41.6) (width 0.2) (layer "F.Cu") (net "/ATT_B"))
 (segment (start 49.8 41.6) (end 56.87 40.33) (width 0.2) (layer "F.Cu") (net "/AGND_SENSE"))
 (segment (start 49.8 41.6) (end 49.8 43.55) (width 0.2) (layer "F.Cu") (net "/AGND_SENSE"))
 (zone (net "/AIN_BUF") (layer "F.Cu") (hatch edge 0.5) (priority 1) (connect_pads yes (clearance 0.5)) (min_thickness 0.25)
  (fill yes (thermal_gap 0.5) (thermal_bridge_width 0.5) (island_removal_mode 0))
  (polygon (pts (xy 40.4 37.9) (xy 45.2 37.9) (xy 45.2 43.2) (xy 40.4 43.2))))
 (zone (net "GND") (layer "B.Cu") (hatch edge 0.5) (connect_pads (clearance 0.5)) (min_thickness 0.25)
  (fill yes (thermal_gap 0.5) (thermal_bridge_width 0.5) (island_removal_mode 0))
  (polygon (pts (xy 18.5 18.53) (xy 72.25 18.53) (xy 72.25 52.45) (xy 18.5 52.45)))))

